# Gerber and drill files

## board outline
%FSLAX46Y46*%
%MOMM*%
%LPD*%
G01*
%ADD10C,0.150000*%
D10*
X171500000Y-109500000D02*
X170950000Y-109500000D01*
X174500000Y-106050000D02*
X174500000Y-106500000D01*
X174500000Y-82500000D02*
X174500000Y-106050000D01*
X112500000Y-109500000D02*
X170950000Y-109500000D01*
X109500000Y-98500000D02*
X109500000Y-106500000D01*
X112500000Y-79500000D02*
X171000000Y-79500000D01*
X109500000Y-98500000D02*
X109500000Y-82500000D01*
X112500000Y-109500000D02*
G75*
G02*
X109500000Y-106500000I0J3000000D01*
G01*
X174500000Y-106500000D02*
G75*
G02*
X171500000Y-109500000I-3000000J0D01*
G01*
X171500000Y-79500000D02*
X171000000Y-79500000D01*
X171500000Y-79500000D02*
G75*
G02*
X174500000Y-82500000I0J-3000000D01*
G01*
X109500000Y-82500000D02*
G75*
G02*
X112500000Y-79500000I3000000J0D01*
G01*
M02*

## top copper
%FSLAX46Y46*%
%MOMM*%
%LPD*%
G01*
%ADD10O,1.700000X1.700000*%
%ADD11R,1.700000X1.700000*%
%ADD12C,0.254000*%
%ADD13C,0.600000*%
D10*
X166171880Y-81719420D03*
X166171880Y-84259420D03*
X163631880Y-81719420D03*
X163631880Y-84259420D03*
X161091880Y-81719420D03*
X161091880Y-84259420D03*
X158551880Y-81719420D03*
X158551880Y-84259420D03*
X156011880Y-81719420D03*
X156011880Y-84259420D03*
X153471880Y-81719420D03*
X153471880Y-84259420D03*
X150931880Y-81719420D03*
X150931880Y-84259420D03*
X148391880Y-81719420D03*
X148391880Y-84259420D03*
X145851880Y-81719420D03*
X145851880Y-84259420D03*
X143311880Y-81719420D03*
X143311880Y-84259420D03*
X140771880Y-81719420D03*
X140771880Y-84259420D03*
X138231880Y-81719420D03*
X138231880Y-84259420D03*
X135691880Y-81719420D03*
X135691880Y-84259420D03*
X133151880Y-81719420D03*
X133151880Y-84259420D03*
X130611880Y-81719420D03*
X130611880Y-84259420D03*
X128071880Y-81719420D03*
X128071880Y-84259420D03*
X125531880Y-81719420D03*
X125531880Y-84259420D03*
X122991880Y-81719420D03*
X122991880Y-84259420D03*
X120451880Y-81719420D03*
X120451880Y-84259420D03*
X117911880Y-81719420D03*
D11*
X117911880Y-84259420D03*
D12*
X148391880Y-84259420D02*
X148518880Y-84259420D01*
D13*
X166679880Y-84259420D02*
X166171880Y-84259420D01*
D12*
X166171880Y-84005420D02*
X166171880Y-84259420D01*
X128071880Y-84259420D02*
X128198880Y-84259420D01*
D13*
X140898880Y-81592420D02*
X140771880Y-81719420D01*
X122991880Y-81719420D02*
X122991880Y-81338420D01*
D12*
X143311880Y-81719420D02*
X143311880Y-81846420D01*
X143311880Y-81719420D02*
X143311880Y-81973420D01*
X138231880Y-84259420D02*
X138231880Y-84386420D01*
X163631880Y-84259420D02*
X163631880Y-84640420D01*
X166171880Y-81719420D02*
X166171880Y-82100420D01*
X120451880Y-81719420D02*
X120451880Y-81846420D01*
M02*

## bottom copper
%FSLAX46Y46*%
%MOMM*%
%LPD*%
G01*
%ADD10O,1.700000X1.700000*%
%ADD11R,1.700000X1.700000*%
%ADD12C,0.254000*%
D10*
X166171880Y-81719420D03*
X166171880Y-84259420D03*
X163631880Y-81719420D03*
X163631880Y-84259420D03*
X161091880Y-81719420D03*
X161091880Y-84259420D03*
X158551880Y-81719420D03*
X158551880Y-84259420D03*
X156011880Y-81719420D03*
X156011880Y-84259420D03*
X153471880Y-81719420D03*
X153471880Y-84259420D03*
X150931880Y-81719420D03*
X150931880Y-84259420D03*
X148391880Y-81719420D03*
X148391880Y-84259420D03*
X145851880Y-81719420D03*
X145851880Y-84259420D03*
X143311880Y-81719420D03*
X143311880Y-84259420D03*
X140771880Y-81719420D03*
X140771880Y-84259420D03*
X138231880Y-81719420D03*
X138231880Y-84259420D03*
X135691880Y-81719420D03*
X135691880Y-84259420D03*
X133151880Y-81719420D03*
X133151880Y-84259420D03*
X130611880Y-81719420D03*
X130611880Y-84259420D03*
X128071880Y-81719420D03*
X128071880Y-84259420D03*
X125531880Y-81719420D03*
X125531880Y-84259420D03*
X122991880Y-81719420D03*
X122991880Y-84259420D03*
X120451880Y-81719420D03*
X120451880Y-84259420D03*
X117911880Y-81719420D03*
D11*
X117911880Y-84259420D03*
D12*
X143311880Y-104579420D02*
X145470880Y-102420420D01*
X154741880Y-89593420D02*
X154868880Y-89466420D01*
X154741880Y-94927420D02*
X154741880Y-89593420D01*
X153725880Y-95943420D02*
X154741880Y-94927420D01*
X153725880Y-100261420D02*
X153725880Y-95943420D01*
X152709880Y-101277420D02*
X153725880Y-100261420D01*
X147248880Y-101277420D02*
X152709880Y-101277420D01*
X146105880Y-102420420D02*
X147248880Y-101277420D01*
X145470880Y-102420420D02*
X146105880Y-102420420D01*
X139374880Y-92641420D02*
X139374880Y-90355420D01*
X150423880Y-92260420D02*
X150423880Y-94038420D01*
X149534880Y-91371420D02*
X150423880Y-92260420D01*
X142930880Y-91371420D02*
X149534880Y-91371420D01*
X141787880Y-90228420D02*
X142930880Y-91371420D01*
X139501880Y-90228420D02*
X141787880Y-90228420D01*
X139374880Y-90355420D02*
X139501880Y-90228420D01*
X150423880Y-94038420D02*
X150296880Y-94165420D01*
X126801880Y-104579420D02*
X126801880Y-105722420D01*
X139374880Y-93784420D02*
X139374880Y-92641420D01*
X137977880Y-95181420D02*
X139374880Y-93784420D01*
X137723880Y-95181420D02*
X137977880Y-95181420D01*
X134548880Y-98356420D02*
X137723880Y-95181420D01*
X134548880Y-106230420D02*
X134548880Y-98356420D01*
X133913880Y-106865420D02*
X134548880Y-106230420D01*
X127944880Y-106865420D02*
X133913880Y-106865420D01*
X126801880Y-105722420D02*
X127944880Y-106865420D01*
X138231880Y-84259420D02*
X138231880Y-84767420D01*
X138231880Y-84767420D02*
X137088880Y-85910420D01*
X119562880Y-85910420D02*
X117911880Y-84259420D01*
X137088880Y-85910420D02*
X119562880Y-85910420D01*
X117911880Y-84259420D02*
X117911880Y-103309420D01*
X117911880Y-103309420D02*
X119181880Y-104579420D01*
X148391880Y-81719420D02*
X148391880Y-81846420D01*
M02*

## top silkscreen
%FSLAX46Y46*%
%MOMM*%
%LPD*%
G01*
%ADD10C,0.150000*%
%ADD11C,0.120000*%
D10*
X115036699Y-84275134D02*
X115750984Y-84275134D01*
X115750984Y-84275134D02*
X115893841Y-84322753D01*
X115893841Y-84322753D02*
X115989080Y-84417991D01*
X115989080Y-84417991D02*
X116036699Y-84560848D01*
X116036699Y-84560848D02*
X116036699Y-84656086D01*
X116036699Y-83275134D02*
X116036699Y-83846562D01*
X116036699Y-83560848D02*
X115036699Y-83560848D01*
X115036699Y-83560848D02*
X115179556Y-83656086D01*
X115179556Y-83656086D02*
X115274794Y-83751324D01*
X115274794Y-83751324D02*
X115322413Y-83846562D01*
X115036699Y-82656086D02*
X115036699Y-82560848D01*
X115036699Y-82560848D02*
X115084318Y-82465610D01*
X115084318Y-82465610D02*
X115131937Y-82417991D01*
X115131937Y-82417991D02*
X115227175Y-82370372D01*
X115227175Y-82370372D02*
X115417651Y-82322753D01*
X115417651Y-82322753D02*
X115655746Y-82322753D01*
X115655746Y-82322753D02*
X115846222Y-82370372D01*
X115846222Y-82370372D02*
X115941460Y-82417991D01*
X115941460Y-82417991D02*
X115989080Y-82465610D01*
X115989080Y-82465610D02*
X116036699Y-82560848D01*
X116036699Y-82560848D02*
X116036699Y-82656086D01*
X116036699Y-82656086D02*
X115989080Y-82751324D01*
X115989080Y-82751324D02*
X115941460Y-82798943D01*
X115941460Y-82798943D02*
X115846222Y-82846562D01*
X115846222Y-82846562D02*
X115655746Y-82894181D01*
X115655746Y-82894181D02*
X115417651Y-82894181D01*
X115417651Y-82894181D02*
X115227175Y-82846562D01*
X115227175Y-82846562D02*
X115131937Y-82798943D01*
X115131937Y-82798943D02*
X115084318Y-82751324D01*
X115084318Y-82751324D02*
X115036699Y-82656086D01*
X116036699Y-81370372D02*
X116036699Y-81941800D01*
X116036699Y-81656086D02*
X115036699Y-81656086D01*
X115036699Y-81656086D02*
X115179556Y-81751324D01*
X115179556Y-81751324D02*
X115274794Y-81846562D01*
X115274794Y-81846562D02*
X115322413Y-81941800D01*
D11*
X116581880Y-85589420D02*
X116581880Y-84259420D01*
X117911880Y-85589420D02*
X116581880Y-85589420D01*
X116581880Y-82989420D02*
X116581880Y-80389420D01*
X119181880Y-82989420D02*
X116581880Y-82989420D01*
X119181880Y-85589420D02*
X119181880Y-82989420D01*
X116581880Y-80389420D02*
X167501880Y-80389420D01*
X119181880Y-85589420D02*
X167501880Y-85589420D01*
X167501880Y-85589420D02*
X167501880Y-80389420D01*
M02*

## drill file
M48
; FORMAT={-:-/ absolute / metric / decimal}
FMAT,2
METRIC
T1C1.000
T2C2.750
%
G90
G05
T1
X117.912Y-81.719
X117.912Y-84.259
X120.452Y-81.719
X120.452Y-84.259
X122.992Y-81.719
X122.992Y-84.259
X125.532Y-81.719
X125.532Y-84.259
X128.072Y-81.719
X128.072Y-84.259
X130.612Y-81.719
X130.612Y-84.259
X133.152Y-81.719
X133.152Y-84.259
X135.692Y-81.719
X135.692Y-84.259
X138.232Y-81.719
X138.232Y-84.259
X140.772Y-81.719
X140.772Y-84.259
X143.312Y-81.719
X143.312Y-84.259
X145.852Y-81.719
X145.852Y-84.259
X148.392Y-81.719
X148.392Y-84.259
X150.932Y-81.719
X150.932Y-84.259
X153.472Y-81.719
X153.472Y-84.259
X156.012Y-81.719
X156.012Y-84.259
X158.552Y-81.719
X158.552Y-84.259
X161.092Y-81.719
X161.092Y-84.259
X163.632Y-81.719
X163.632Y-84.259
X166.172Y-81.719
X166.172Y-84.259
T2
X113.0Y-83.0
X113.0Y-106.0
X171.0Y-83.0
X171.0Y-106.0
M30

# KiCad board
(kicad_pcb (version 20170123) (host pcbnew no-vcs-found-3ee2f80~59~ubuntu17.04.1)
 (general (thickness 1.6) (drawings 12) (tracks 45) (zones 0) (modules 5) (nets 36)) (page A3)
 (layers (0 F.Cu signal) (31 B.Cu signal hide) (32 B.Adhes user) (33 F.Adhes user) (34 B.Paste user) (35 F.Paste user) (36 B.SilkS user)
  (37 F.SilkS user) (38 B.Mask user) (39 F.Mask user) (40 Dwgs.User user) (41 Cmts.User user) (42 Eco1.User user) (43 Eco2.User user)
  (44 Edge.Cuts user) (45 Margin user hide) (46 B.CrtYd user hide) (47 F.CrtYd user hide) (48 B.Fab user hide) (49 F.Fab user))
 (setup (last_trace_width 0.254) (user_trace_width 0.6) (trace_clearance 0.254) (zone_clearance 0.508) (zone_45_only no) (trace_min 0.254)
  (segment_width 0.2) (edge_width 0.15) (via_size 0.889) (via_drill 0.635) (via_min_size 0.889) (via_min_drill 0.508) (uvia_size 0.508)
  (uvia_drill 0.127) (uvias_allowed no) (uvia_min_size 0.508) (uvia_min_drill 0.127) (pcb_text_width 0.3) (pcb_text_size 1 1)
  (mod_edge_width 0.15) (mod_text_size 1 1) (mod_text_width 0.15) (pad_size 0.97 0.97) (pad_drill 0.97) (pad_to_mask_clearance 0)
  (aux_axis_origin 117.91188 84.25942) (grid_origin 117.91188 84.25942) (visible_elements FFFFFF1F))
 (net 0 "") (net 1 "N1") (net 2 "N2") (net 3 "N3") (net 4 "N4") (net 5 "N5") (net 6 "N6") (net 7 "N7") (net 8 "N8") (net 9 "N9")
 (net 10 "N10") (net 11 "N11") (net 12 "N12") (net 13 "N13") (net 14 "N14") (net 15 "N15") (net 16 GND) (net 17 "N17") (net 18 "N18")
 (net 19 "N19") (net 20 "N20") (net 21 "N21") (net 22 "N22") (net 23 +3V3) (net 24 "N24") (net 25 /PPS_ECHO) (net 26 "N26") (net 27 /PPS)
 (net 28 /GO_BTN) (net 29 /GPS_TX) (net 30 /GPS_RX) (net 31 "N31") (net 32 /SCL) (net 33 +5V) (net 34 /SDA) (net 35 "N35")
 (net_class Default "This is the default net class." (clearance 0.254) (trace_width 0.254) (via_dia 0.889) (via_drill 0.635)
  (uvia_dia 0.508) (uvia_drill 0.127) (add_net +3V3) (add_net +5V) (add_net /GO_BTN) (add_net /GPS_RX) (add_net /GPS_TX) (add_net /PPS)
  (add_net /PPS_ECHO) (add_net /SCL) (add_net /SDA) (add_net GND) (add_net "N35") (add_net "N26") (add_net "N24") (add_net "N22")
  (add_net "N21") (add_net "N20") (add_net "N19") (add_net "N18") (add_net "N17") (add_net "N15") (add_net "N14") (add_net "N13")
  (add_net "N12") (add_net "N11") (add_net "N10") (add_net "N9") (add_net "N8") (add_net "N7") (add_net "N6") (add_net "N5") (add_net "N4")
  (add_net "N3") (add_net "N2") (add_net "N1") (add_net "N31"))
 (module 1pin (layer F.Cu) (at 171 106)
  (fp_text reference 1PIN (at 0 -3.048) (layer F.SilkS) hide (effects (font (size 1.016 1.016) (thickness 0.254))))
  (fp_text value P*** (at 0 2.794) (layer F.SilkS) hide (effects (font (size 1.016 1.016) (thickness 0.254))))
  (pad "" np_thru_hole circle (at 0 0) (size 2.75 2.75) (drill 2.75) (layers *.Cu)))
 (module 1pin (layer F.Cu) (at 113 106)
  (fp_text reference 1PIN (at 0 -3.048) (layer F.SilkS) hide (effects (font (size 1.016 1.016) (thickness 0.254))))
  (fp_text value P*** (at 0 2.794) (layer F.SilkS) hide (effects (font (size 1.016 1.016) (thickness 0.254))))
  (pad "" np_thru_hole circle (at 0 0) (size 2.75 2.75) (drill 2.75) (layers *.Cu)))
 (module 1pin (layer F.Cu) (at 171 83)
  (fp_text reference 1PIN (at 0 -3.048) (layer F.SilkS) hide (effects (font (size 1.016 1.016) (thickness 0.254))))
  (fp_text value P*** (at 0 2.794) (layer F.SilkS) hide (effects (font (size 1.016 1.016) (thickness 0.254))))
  (pad "" np_thru_hole circle (at 0 0) (size 2.75 2.75) (drill 2.75) (layers *.Cu)))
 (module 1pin (layer F.Cu) (at 113 83)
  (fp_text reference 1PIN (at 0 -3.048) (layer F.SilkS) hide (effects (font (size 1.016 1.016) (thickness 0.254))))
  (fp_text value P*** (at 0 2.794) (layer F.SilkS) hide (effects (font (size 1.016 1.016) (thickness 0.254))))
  (pad "" np_thru_hole circle (at 0 0) (size 2.75 2.75) (drill 2.75) (layers *.Cu)))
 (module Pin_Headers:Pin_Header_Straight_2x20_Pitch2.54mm (layer F.Cu) (at 117.91188 84.25942 90)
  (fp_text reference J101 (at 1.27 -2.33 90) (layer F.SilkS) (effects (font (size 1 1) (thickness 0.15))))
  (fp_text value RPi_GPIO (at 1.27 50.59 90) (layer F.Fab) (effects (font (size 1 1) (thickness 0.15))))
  (fp_line (start -1.33 -1.33) (end 0 -1.33) (layer F.SilkS) (width 0.12))
  (fp_line (start -1.33 0) (end -1.33 -1.33) (layer F.SilkS) (width 0.12))
  (fp_line (start 1.27 -1.33) (end 3.87 -1.33) (layer F.SilkS) (width 0.12))
  (fp_line (start 1.27 1.27) (end 1.27 -1.33) (layer F.SilkS) (width 0.12))
  (fp_line (start -1.33 1.27) (end 1.27 1.27) (layer F.SilkS) (width 0.12))
  (fp_line (start 3.87 -1.33) (end 3.87 49.59) (layer F.SilkS) (width 0.12))
  (fp_line (start -1.33 1.27) (end -1.33 49.59) (layer F.SilkS) (width 0.12))
  (fp_line (start -1.33 49.59) (end 3.87 49.59) (layer F.SilkS) (width 0.12))
  (pad 40 thru_hole oval (at 2.54 48.26 90) (size 1.7 1.7) (drill 1) (layers *.Cu *.Mask) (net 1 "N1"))
  (pad 39 thru_hole oval (at 0 48.26 90) (size 1.7 1.7) (drill 1) (layers *.Cu *.Mask) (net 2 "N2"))
  (pad 38 thru_hole oval (at 2.54 45.72 90) (size 1.7 1.7) (drill 1) (layers *.Cu *.Mask) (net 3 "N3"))
  (pad 37 thru_hole oval (at 0 45.72 90) (size 1.7 1.7) (drill 1) (layers *.Cu *.Mask) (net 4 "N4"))
  (pad 36 thru_hole oval (at 2.54 43.18 90) (size 1.7 1.7) (drill 1) (layers *.Cu *.Mask) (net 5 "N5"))
  (pad 35 thru_hole oval (at 0 43.18 90) (size 1.7 1.7) (drill 1) (layers *.Cu *.Mask) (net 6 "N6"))
  (pad 34 thru_hole oval (at 2.54 40.64 90) (size 1.7 1.7) (drill 1) (layers *.Cu *.Mask) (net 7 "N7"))
  (pad 33 thru_hole oval (at 0 40.64 90) (size 1.7 1.7) (drill 1) (layers *.Cu *.Mask) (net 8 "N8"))
  (pad 32 thru_hole oval (at 2.54 38.1 90) (size 1.7 1.7) (drill 1) (layers *.Cu *.Mask) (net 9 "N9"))
  (pad 31 thru_hole oval (at 0 38.1 90) (size 1.7 1.7) (drill 1) (layers *.Cu *.Mask) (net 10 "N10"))
  (pad 30 thru_hole oval (at 2.54 35.56 90) (size 1.7 1.7) (drill 1) (layers *.Cu *.Mask) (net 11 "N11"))
  (pad 29 thru_hole oval (at 0 35.56 90) (size 1.7 1.7) (drill 1) (layers *.Cu *.Mask) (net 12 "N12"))
  (pad 28 thru_hole oval (at 2.54 33.02 90) (size 1.7 1.7) (drill 1) (layers *.Cu *.Mask) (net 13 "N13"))
  (pad 27 thru_hole oval (at 0 33.02 90) (size 1.7 1.7) (drill 1) (layers *.Cu *.Mask) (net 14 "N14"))
  (pad 26 thru_hole oval (at 2.54 30.48 90) (size 1.7 1.7) (drill 1) (layers *.Cu *.Mask) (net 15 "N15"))
  (pad 25 thru_hole oval (at 0 30.48 90) (size 1.7 1.7) (drill 1) (layers *.Cu *.Mask) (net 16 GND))
  (pad 24 thru_hole oval (at 2.54 27.94 90) (size 1.7 1.7) (drill 1) (layers *.Cu *.Mask) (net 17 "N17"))
  (pad 23 thru_hole oval (at 0 27.94 90) (size 1.7 1.7) (drill 1) (layers *.Cu *.Mask) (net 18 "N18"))
  (pad 22 thru_hole oval (at 2.54 25.4 90) (size 1.7 1.7) (drill 1) (layers *.Cu *.Mask) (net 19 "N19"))
  (pad 21 thru_hole oval (at 0 25.4 90) (size 1.7 1.7) (drill 1) (layers *.Cu *.Mask) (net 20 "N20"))
  (pad 20 thru_hole oval (at 2.54 22.86 90) (size 1.7 1.7) (drill 1) (layers *.Cu *.Mask) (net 16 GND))
  (pad 19 thru_hole oval (at 0 22.86 90) (size 1.7 1.7) (drill 1) (layers *.Cu *.Mask) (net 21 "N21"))
  (pad 18 thru_hole oval (at 2.54 20.32 90) (size 1.7 1.7) (drill 1) (layers *.Cu *.Mask) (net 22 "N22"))
  (pad 17 thru_hole oval (at 0 20.32 90) (size 1.7 1.7) (drill 1) (layers *.Cu *.Mask) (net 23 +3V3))
  (pad 16 thru_hole oval (at 2.54 17.78 90) (size 1.7 1.7) (drill 1) (layers *.Cu *.Mask) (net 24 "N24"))
  (pad 15 thru_hole oval (at 0 17.78 90) (size 1.7 1.7) (drill 1) (layers *.Cu *.Mask) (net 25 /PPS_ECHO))
  (pad 14 thru_hole oval (at 2.54 15.24 90) (size 1.7 1.7) (drill 1) (layers *.Cu *.Mask) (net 16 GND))
  (pad 13 thru_hole oval (at 0 15.24 90) (size 1.7 1.7) (drill 1) (layers *.Cu *.Mask) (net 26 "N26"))
  (pad 12 thru_hole oval (at 2.54 12.7 90) (size 1.7 1.7) (drill 1) (layers *.Cu *.Mask) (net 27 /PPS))
  (pad 11 thru_hole oval (at 0 12.7 90) (size 1.7 1.7) (drill 1) (layers *.Cu *.Mask) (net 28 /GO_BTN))
  (pad 10 thru_hole oval (at 2.54 10.16 90) (size 1.7 1.7) (drill 1) (layers *.Cu *.Mask) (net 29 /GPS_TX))
  (pad 9 thru_hole oval (at 0 10.16 90) (size 1.7 1.7) (drill 1) (layers *.Cu *.Mask) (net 16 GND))
  (pad 8 thru_hole oval (at 2.54 7.62 90) (size 1.7 1.7) (drill 1) (layers *.Cu *.Mask) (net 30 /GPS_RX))
  (pad 7 thru_hole oval (at 0 7.62 90) (size 1.7 1.7) (drill 1) (layers *.Cu *.Mask) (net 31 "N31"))
  (pad 6 thru_hole oval (at 2.54 5.08 90) (size 1.7 1.7) (drill 1) (layers *.Cu *.Mask) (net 16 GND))
  (pad 5 thru_hole oval (at 0 5.08 90) (size 1.7 1.7) (drill 1) (layers *.Cu *.Mask) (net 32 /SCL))
  (pad 4 thru_hole oval (at 2.54 2.54 90) (size 1.7 1.7) (drill 1) (layers *.Cu *.Mask) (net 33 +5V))
  (pad 3 thru_hole oval (at 0 2.54 90) (size 1.7 1.7) (drill 1) (layers *.Cu *.Mask) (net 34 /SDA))
  (pad 2 thru_hole oval (at 2.54 0 90) (size 1.7 1.7) (drill 1) (layers *.Cu *.Mask) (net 33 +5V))
  (pad 1 thru_hole rect (at 0 0 90) (size 1.7 1.7) (drill 1) (layers *.Cu *.Mask) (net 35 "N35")))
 (gr_line (start 171.5 109.5) (end 170.95 109.5) (angle 90) (layer Edge.Cuts) (width 0.15))
 (gr_line (start 174.5 106.05) (end 174.5 106.5) (angle 90) (layer Edge.Cuts) (width 0.15))
 (gr_line (start 174.5 82.5) (end 174.5 106.05) (angle 90) (layer Edge.Cuts) (width 0.15))
 (gr_line (start 112.5 109.5) (end 170.95 109.5) (angle 90) (layer Edge.Cuts) (width 0.15))
 (gr_line (start 109.5 98.5) (end 109.5 106.5) (angle 90) (layer Edge.Cuts) (width 0.15))
 (gr_line (start 112.5 79.5) (end 171 79.5) (angle 90) (layer Edge.Cuts) (width 0.15))
 (gr_line (start 109.5 98.5) (end 109.5 82.5) (angle 90) (layer Edge.Cuts) (width 0.15))
 (gr_arc (start 112.5 106.5) (end 112.5 109.5) (angle 90) (layer Edge.Cuts) (width 0.15))
 (gr_arc (start 171.5 106.5) (end 174.5 106.5) (angle 90) (layer Edge.Cuts) (width 0.15))
 (gr_line (start 171.5 79.5) (end 171 79.5) (angle 90) (layer Edge.Cuts) (width 0.15))
 (gr_arc (start 171.5 82.5) (end 171.5 79.5) (angle 90) (layer Edge.Cuts) (width 0.15))
 (gr_arc (start 112.5 82.5) (end 109.5 82.5) (angle 90) (layer Edge.Cuts) (width 0.15))
 (segment (start 143.31188 104.57942) (end 145.47088 102.42042) (width 0.254) (layer B.Cu) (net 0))
 (segment (start 154.74188 89.59342) (end 154.86888 89.46642) (width 0.254) (layer B.Cu) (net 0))
 (segment (start 154.74188 94.92742) (end 154.74188 89.59342) (width 0.254) (layer B.Cu) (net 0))
 (segment (start 153.72588 95.94342) (end 154.74188 94.92742) (width 0.254) (layer B.Cu) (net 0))
 (segment (start 153.72588 100.26142) (end 153.72588 95.94342) (width 0.254) (layer B.Cu) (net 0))
 (segment (start 152.70988 101.27742) (end 153.72588 100.26142) (width 0.254) (layer B.Cu) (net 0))
 (segment (start 147.24888 101.27742) (end 152.70988 101.27742) (width 0.254) (layer B.Cu) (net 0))
 (segment (start 146.10588 102.42042) (end 147.24888 101.27742) (width 0.254) (layer B.Cu) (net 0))
 (segment (start 145.47088 102.42042) (end 146.10588 102.42042) (width 0.254) (layer B.Cu) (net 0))
 (segment (start 139.37488 92.64142) (end 139.37488 90.35542) (width 0.254) (layer B.Cu) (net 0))
 (segment (start 150.42388 92.26042) (end 150.42388 94.03842) (width 0.254) (layer B.Cu) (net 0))
 (segment (start 149.53488 91.37142) (end 150.42388 92.26042) (width 0.254) (layer B.Cu) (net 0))
 (segment (start 142.93088 91.37142) (end 149.53488 91.37142) (width 0.254) (layer B.Cu) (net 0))
 (segment (start 141.78788 90.22842) (end 142.93088 91.37142) (width 0.254) (layer B.Cu) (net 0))
 (segment (start 139.50188 90.22842) (end 141.78788 90.22842) (width 0.254) (layer B.Cu) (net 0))
 (segment (start 139.37488 90.35542) (end 139.50188 90.22842) (width 0.254) (layer B.Cu) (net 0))
 (segment (start 150.42388 94.03842) (end 150.29688 94.16542) (width 0.254) (layer B.Cu) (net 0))
 (segment (start 126.80188 104.57942) (end 126.80188 105.72242) (width 0.254) (layer B.Cu) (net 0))
 (segment (start 139.37488 93.78442) (end 139.37488 92.64142) (width 0.254) (layer B.Cu) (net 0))
 (segment (start 137.97788 95.18142) (end 139.37488 93.78442) (width 0.254) (layer B.Cu) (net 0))
 (segment (start 137.72388 95.18142) (end 137.97788 95.18142) (width 0.254) (layer B.Cu) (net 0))
 (segment (start 134.54888 98.35642) (end 137.72388 95.18142) (width 0.254) (layer B.Cu) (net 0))
 (segment (start 134.54888 106.23042) (end 134.54888 98.35642) (width 0.254) (layer B.Cu) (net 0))
 (segment (start 133.91388 106.86542) (end 134.54888 106.23042) (width 0.254) (layer B.Cu) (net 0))
 (segment (start 127.94488 106.86542) (end 133.91388 106.86542) (width 0.254) (layer B.Cu) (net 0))
 (segment (start 126.80188 105.72242) (end 127.94488 106.86542) (width 0.254) (layer B.Cu) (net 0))
 (segment (start 148.39188 84.25942) (end 148.51888 84.25942) (width 0.254) (layer F.Cu) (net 16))
 (segment (start 166.67988 84.25942) (end 166.17188 84.25942) (width 0.6) (layer F.Cu) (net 2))
 (segment (start 166.17188 84.00542) (end 166.17188 84.25942) (width 0.254) (layer F.Cu) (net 2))
 (segment (start 128.07188 84.25942) (end 128.19888 84.25942) (width 0.254) (layer F.Cu) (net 16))
 (segment (start 140.89888 81.59242) (end 140.77188 81.71942) (width 0.6) (layer F.Cu) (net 16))
 (segment (start 122.99188 81.71942) (end 122.99188 81.33842) (width 0.6) (layer F.Cu) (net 16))
 (segment (start 143.31188 81.71942) (end 143.31188 81.84642) (width 0.254) (layer F.Cu) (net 19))
 (segment (start 143.31188 81.71942) (end 143.31188 81.97342) (width 0.254) (layer F.Cu) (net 19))
 (segment (start 138.23188 84.25942) (end 138.23188 84.76742) (width 0.254) (layer B.Cu) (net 23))
 (segment (start 138.23188 84.76742) (end 137.08888 85.91042) (width 0.254) (layer B.Cu) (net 23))
 (segment (start 119.56288 85.91042) (end 117.91188 84.25942) (width 0.254) (layer B.Cu) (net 23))
 (segment (start 137.08888 85.91042) (end 119.56288 85.91042) (width 0.254) (layer B.Cu) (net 23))
 (segment (start 117.91188 84.25942) (end 117.91188 103.30942) (width 0.254) (layer B.Cu) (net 23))
 (segment (start 117.91188 103.30942) (end 119.18188 104.57942) (width 0.254) (layer B.Cu) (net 23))
 (segment (start 138.23188 84.25942) (end 138.23188 84.38642) (width 0.254) (layer F.Cu) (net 23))
 (segment (start 163.63188 84.25942) (end 163.63188 84.64042) (width 0.254) (layer F.Cu) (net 4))
 (segment (start 166.17188 81.71942) (end 166.17188 82.10042) (width 0.254) (layer F.Cu) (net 1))
 (segment (start 148.39188 81.71942) (end 148.39188 81.84642) (width 0.254) (layer B.Cu) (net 15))
 (segment (start 120.45188 81.71942) (end 120.45188 81.84642) (width 0.254) (layer F.Cu) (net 33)))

